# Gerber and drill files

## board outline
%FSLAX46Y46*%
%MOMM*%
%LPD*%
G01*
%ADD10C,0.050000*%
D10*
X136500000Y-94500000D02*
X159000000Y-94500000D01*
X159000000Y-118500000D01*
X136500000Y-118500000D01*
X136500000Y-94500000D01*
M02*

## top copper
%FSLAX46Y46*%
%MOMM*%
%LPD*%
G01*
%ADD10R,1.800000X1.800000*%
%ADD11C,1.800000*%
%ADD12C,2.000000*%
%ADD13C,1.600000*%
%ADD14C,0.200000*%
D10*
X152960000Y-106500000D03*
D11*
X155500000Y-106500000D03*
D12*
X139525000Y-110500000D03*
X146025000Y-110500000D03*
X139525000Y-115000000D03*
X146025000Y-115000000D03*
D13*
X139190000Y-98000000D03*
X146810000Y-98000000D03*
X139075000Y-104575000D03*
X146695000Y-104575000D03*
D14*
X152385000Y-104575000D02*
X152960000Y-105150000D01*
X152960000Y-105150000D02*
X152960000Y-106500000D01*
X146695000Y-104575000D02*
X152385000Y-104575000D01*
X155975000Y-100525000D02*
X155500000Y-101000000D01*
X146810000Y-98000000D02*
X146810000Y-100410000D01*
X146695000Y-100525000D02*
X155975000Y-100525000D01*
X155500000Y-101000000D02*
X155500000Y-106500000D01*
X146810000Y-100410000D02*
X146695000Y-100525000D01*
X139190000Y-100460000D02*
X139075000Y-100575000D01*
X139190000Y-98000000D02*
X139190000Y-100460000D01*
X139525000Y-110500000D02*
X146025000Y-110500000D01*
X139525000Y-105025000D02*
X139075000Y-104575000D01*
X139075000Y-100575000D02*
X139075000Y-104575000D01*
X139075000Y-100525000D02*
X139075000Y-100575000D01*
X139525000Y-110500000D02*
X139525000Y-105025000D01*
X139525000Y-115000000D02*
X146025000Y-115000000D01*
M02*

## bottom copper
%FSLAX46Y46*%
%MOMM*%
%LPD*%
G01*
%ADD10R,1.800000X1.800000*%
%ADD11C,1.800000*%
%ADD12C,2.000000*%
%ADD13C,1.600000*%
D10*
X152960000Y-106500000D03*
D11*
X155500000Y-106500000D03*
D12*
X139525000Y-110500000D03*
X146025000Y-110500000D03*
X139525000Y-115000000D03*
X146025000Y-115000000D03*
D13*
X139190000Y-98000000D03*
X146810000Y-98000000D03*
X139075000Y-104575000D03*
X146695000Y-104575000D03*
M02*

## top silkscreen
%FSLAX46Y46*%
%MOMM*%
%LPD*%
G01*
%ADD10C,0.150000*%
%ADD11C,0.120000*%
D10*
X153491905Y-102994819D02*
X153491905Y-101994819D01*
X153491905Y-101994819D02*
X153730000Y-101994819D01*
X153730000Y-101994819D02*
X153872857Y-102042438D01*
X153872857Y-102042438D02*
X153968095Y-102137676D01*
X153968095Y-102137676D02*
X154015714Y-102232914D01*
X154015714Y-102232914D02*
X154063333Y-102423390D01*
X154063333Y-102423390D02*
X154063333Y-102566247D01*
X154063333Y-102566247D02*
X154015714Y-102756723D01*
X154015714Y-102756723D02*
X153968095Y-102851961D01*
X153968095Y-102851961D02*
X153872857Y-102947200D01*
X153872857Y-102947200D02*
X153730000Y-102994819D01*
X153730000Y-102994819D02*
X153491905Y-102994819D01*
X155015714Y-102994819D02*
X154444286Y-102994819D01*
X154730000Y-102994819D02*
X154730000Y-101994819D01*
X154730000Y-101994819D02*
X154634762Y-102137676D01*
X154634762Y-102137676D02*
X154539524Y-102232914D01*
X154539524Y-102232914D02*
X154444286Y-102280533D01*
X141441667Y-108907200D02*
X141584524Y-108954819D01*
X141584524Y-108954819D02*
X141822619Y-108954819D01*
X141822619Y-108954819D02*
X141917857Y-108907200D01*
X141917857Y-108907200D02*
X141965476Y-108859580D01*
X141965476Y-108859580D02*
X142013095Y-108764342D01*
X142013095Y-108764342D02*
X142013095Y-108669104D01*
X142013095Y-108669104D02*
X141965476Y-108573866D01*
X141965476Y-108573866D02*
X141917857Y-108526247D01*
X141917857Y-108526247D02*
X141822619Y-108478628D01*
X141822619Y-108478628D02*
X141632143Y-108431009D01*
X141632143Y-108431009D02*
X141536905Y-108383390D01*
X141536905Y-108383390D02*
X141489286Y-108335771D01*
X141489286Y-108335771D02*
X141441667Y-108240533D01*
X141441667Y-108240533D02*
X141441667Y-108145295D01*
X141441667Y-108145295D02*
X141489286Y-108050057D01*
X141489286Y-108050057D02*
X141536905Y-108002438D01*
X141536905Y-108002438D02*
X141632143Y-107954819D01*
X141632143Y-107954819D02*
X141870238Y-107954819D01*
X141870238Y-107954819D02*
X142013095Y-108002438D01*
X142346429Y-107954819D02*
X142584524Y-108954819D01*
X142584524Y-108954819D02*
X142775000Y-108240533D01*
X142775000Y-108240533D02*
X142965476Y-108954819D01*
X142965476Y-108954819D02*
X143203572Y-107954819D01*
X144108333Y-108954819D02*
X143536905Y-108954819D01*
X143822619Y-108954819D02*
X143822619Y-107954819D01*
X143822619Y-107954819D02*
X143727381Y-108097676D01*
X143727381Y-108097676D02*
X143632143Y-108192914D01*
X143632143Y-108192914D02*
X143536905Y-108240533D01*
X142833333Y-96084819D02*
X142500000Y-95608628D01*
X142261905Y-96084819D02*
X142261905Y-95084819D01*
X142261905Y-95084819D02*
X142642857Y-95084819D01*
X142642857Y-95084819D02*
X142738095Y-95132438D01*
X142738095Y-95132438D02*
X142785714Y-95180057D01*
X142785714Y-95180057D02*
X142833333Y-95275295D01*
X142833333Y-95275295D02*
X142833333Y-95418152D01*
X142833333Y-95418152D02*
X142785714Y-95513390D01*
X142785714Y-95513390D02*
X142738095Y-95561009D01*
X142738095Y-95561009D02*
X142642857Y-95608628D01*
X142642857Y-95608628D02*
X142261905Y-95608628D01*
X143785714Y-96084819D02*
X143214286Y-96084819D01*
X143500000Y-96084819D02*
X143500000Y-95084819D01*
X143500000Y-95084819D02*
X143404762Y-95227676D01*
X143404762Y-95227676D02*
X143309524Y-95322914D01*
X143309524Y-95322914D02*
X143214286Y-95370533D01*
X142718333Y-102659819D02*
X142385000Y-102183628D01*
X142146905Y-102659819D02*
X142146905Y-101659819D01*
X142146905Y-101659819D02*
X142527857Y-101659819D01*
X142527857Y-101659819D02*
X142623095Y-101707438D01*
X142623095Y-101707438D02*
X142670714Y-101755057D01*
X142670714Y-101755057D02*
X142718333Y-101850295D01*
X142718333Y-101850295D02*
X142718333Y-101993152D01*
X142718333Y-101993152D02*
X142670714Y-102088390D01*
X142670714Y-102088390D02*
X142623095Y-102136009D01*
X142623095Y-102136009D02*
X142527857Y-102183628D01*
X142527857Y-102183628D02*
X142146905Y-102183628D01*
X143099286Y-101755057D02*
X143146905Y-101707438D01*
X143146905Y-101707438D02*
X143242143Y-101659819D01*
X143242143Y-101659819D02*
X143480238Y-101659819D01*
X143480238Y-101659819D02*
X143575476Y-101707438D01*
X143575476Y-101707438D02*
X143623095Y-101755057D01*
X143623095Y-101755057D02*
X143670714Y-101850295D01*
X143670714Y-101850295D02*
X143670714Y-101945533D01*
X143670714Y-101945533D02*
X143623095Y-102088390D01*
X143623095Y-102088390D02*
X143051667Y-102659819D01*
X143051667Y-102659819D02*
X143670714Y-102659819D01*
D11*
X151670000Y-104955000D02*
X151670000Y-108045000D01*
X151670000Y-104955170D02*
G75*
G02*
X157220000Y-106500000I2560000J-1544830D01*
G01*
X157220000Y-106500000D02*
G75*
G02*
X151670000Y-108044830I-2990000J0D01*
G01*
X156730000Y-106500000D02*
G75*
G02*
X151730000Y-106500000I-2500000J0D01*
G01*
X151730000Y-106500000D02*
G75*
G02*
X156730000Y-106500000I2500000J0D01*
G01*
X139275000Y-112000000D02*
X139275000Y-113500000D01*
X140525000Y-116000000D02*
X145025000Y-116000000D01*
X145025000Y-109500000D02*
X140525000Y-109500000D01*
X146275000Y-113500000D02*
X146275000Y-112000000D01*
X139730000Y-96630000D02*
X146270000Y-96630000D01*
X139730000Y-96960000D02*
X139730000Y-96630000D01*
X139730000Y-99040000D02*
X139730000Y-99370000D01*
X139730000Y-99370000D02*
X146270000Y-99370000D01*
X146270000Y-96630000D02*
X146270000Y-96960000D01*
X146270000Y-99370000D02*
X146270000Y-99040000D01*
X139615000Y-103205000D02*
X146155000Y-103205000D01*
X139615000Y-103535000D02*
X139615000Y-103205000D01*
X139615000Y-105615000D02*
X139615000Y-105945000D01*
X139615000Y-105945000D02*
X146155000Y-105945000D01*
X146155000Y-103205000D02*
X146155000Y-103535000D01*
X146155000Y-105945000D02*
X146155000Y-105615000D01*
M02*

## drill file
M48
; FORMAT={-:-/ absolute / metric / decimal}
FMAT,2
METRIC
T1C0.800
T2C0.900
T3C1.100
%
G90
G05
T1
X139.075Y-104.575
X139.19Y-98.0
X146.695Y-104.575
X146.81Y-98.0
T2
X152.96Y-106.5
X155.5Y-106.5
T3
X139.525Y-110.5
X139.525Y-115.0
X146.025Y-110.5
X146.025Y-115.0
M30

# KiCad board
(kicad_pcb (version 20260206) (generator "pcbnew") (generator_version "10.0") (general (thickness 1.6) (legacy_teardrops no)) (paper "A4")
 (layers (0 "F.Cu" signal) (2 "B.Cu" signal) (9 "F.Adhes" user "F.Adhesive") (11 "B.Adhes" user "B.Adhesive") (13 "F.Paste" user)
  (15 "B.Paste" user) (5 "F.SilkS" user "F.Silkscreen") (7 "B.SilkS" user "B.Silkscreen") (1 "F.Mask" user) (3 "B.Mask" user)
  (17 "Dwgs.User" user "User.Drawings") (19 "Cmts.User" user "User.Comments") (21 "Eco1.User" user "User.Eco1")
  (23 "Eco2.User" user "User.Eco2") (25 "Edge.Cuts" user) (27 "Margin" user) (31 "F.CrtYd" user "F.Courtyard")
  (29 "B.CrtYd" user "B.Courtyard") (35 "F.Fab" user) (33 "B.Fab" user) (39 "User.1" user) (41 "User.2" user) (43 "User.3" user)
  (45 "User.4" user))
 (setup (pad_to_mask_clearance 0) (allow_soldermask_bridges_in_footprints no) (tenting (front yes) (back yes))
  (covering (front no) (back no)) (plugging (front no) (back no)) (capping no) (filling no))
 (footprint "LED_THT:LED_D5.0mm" (layer "F.Cu") (at 152.96 106.5)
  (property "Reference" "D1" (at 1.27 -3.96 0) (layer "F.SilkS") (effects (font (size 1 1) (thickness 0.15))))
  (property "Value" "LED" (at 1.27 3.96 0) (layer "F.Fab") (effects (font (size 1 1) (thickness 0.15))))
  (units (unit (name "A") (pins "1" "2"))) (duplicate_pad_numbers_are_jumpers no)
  (fp_line (start -1.29 -1.545) (end -1.29 1.545) (stroke (width 0.12) (type solid)) (layer "F.SilkS"))
  (fp_arc (start -1.29 -1.54483) (mid 2.071779 -2.880495) (end 4.26 0) (stroke (width 0.12) (type solid)) (layer "F.SilkS"))
  (fp_arc (start 4.26 0) (mid 2.071779 2.880495) (end -1.29 1.54483) (stroke (width 0.12) (type solid)) (layer "F.SilkS"))
  (fp_circle (center 1.27 0) (end 3.77 0) (stroke (width 0.12) (type solid)) (fill no) (layer "F.SilkS"))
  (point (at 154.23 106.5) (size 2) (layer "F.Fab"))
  (pad "1" thru_hole rect (at 0 0) (size 1.8 1.8) (drill 0.9) (layers "*.Cu" "*.Mask") (remove_unused_layers no) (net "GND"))
  (pad "2" thru_hole circle (at 2.54 0) (size 1.8 1.8) (drill 0.9) (layers "*.Cu" "*.Mask") (remove_unused_layers no) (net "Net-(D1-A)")))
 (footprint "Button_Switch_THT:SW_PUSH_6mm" (layer "F.Cu") (at 139.525 110.5)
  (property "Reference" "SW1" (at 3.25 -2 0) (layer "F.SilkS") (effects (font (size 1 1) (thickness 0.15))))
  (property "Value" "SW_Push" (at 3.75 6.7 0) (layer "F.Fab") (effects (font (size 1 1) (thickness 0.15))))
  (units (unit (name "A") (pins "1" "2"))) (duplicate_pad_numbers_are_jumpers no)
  (fp_line (start -0.25 1.5) (end -0.25 3) (stroke (width 0.12) (type solid)) (layer "F.SilkS"))
  (fp_line (start 1 5.5) (end 5.5 5.5) (stroke (width 0.12) (type solid)) (layer "F.SilkS"))
  (fp_line (start 5.5 -1) (end 1 -1) (stroke (width 0.12) (type solid)) (layer "F.SilkS"))
  (fp_line (start 6.75 3) (end 6.75 1.5) (stroke (width 0.12) (type solid)) (layer "F.SilkS"))
  (pad "1" thru_hole circle (at 0 0 90) (size 2 2) (drill 1.1) (layers "*.Cu" "*.Mask") (remove_unused_layers no) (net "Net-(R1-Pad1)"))
  (pad "1" thru_hole circle (at 6.5 0 90) (size 2 2) (drill 1.1) (layers "*.Cu" "*.Mask") (remove_unused_layers no) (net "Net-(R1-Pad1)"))
  (pad "2" thru_hole circle (at 0 4.5 90) (size 2 2) (drill 1.1) (layers "*.Cu" "*.Mask") (remove_unused_layers no) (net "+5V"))
  (pad "2" thru_hole circle (at 6.5 4.5 90) (size 2 2) (drill 1.1) (layers "*.Cu" "*.Mask") (remove_unused_layers no) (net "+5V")))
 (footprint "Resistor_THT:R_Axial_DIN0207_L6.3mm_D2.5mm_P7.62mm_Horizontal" (layer "F.Cu") (at 139.19 98)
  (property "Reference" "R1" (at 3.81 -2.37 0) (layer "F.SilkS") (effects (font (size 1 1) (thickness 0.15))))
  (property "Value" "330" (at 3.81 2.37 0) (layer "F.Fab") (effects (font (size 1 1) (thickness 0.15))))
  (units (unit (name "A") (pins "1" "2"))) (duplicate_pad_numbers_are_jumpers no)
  (fp_line (start 0.54 -1.37) (end 7.08 -1.37) (stroke (width 0.12) (type solid)) (layer "F.SilkS"))
  (fp_line (start 0.54 -1.04) (end 0.54 -1.37) (stroke (width 0.12) (type solid)) (layer "F.SilkS"))
  (fp_line (start 0.54 1.04) (end 0.54 1.37) (stroke (width 0.12) (type solid)) (layer "F.SilkS"))
  (fp_line (start 0.54 1.37) (end 7.08 1.37) (stroke (width 0.12) (type solid)) (layer "F.SilkS"))
  (fp_line (start 7.08 -1.37) (end 7.08 -1.04) (stroke (width 0.12) (type solid)) (layer "F.SilkS"))
  (fp_line (start 7.08 1.37) (end 7.08 1.04) (stroke (width 0.12) (type solid)) (layer "F.SilkS"))
  (pad "1" thru_hole circle (at 0 0) (size 1.6 1.6) (drill 0.8) (layers "*.Cu" "*.Mask") (remove_unused_layers no) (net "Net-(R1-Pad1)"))
  (pad "2" thru_hole circle (at 7.62 0) (size 1.6 1.6) (drill 0.8) (layers "*.Cu" "*.Mask") (remove_unused_layers no) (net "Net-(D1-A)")))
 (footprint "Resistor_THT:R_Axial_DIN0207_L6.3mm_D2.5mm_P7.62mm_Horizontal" (layer "F.Cu") (at 139.075 104.575)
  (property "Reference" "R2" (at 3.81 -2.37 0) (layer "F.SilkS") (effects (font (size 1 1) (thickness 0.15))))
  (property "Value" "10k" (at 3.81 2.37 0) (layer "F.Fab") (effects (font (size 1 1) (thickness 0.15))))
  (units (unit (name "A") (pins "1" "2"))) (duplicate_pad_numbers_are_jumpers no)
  (fp_line (start 0.54 -1.37) (end 7.08 -1.37) (stroke (width 0.12) (type solid)) (layer "F.SilkS"))
  (fp_line (start 0.54 -1.04) (end 0.54 -1.37) (stroke (width 0.12) (type solid)) (layer "F.SilkS"))
  (fp_line (start 0.54 1.04) (end 0.54 1.37) (stroke (width 0.12) (type solid)) (layer "F.SilkS"))
  (fp_line (start 0.54 1.37) (end 7.08 1.37) (stroke (width 0.12) (type solid)) (layer "F.SilkS"))
  (fp_line (start 7.08 -1.37) (end 7.08 -1.04) (stroke (width 0.12) (type solid)) (layer "F.SilkS"))
  (fp_line (start 7.08 1.37) (end 7.08 1.04) (stroke (width 0.12) (type solid)) (layer "F.SilkS"))
  (pad "1" thru_hole circle (at 0 0) (size 1.6 1.6) (drill 0.8) (layers "*.Cu" "*.Mask") (remove_unused_layers no) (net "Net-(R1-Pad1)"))
  (pad "2" thru_hole circle (at 7.62 0) (size 1.6 1.6) (drill 0.8) (layers "*.Cu" "*.Mask") (remove_unused_layers no) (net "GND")))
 (gr_rect (start 136.5 94.5) (end 159 118.5) (stroke (width 0.05) (type default)) (fill no) (layer "Edge.Cuts"))
 (segment (start 152.385 104.575) (end 152.96 105.15) (width 0.2) (layer "F.Cu") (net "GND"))
 (segment (start 152.96 105.15) (end 152.96 106.5) (width 0.2) (layer "F.Cu") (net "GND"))
 (segment (start 146.695 104.575) (end 152.385 104.575) (width 0.2) (layer "F.Cu") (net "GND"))
 (segment (start 155.975 100.525) (end 155.5 101) (width 0.2) (layer "F.Cu") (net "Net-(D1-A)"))
 (segment (start 146.81 98) (end 146.81 100.41) (width 0.2) (layer "F.Cu") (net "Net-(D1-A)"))
 (segment (start 146.695 100.525) (end 155.975 100.525) (width 0.2) (layer "F.Cu") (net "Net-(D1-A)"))
 (segment (start 155.5 101) (end 155.5 106.5) (width 0.2) (layer "F.Cu") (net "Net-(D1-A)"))
 (segment (start 146.81 100.41) (end 146.695 100.525) (width 0.2) (layer "F.Cu") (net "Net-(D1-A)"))
 (segment (start 139.19 100.46) (end 139.075 100.575) (width 0.2) (layer "F.Cu") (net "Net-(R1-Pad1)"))
 (segment (start 139.19 98) (end 139.19 100.46) (width 0.2) (layer "F.Cu") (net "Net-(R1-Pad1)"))
 (segment (start 139.525 110.5) (end 146.025 110.5) (width 0.2) (layer "F.Cu") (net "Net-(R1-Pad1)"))
 (segment (start 139.525 105.025) (end 139.075 104.575) (width 0.2) (layer "F.Cu") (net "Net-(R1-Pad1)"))
 (segment (start 139.075 100.575) (end 139.075 104.575) (width 0.2) (layer "F.Cu") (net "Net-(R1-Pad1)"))
 (segment (start 139.075 100.525) (end 139.075 100.575) (width 0.2) (layer "F.Cu") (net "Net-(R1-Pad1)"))
 (segment (start 139.525 110.5) (end 139.525 105.025) (width 0.2) (layer "F.Cu") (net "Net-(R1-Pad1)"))
 (segment (start 139.525 115) (end 146.025 115) (width 0.2) (layer "F.Cu") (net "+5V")))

